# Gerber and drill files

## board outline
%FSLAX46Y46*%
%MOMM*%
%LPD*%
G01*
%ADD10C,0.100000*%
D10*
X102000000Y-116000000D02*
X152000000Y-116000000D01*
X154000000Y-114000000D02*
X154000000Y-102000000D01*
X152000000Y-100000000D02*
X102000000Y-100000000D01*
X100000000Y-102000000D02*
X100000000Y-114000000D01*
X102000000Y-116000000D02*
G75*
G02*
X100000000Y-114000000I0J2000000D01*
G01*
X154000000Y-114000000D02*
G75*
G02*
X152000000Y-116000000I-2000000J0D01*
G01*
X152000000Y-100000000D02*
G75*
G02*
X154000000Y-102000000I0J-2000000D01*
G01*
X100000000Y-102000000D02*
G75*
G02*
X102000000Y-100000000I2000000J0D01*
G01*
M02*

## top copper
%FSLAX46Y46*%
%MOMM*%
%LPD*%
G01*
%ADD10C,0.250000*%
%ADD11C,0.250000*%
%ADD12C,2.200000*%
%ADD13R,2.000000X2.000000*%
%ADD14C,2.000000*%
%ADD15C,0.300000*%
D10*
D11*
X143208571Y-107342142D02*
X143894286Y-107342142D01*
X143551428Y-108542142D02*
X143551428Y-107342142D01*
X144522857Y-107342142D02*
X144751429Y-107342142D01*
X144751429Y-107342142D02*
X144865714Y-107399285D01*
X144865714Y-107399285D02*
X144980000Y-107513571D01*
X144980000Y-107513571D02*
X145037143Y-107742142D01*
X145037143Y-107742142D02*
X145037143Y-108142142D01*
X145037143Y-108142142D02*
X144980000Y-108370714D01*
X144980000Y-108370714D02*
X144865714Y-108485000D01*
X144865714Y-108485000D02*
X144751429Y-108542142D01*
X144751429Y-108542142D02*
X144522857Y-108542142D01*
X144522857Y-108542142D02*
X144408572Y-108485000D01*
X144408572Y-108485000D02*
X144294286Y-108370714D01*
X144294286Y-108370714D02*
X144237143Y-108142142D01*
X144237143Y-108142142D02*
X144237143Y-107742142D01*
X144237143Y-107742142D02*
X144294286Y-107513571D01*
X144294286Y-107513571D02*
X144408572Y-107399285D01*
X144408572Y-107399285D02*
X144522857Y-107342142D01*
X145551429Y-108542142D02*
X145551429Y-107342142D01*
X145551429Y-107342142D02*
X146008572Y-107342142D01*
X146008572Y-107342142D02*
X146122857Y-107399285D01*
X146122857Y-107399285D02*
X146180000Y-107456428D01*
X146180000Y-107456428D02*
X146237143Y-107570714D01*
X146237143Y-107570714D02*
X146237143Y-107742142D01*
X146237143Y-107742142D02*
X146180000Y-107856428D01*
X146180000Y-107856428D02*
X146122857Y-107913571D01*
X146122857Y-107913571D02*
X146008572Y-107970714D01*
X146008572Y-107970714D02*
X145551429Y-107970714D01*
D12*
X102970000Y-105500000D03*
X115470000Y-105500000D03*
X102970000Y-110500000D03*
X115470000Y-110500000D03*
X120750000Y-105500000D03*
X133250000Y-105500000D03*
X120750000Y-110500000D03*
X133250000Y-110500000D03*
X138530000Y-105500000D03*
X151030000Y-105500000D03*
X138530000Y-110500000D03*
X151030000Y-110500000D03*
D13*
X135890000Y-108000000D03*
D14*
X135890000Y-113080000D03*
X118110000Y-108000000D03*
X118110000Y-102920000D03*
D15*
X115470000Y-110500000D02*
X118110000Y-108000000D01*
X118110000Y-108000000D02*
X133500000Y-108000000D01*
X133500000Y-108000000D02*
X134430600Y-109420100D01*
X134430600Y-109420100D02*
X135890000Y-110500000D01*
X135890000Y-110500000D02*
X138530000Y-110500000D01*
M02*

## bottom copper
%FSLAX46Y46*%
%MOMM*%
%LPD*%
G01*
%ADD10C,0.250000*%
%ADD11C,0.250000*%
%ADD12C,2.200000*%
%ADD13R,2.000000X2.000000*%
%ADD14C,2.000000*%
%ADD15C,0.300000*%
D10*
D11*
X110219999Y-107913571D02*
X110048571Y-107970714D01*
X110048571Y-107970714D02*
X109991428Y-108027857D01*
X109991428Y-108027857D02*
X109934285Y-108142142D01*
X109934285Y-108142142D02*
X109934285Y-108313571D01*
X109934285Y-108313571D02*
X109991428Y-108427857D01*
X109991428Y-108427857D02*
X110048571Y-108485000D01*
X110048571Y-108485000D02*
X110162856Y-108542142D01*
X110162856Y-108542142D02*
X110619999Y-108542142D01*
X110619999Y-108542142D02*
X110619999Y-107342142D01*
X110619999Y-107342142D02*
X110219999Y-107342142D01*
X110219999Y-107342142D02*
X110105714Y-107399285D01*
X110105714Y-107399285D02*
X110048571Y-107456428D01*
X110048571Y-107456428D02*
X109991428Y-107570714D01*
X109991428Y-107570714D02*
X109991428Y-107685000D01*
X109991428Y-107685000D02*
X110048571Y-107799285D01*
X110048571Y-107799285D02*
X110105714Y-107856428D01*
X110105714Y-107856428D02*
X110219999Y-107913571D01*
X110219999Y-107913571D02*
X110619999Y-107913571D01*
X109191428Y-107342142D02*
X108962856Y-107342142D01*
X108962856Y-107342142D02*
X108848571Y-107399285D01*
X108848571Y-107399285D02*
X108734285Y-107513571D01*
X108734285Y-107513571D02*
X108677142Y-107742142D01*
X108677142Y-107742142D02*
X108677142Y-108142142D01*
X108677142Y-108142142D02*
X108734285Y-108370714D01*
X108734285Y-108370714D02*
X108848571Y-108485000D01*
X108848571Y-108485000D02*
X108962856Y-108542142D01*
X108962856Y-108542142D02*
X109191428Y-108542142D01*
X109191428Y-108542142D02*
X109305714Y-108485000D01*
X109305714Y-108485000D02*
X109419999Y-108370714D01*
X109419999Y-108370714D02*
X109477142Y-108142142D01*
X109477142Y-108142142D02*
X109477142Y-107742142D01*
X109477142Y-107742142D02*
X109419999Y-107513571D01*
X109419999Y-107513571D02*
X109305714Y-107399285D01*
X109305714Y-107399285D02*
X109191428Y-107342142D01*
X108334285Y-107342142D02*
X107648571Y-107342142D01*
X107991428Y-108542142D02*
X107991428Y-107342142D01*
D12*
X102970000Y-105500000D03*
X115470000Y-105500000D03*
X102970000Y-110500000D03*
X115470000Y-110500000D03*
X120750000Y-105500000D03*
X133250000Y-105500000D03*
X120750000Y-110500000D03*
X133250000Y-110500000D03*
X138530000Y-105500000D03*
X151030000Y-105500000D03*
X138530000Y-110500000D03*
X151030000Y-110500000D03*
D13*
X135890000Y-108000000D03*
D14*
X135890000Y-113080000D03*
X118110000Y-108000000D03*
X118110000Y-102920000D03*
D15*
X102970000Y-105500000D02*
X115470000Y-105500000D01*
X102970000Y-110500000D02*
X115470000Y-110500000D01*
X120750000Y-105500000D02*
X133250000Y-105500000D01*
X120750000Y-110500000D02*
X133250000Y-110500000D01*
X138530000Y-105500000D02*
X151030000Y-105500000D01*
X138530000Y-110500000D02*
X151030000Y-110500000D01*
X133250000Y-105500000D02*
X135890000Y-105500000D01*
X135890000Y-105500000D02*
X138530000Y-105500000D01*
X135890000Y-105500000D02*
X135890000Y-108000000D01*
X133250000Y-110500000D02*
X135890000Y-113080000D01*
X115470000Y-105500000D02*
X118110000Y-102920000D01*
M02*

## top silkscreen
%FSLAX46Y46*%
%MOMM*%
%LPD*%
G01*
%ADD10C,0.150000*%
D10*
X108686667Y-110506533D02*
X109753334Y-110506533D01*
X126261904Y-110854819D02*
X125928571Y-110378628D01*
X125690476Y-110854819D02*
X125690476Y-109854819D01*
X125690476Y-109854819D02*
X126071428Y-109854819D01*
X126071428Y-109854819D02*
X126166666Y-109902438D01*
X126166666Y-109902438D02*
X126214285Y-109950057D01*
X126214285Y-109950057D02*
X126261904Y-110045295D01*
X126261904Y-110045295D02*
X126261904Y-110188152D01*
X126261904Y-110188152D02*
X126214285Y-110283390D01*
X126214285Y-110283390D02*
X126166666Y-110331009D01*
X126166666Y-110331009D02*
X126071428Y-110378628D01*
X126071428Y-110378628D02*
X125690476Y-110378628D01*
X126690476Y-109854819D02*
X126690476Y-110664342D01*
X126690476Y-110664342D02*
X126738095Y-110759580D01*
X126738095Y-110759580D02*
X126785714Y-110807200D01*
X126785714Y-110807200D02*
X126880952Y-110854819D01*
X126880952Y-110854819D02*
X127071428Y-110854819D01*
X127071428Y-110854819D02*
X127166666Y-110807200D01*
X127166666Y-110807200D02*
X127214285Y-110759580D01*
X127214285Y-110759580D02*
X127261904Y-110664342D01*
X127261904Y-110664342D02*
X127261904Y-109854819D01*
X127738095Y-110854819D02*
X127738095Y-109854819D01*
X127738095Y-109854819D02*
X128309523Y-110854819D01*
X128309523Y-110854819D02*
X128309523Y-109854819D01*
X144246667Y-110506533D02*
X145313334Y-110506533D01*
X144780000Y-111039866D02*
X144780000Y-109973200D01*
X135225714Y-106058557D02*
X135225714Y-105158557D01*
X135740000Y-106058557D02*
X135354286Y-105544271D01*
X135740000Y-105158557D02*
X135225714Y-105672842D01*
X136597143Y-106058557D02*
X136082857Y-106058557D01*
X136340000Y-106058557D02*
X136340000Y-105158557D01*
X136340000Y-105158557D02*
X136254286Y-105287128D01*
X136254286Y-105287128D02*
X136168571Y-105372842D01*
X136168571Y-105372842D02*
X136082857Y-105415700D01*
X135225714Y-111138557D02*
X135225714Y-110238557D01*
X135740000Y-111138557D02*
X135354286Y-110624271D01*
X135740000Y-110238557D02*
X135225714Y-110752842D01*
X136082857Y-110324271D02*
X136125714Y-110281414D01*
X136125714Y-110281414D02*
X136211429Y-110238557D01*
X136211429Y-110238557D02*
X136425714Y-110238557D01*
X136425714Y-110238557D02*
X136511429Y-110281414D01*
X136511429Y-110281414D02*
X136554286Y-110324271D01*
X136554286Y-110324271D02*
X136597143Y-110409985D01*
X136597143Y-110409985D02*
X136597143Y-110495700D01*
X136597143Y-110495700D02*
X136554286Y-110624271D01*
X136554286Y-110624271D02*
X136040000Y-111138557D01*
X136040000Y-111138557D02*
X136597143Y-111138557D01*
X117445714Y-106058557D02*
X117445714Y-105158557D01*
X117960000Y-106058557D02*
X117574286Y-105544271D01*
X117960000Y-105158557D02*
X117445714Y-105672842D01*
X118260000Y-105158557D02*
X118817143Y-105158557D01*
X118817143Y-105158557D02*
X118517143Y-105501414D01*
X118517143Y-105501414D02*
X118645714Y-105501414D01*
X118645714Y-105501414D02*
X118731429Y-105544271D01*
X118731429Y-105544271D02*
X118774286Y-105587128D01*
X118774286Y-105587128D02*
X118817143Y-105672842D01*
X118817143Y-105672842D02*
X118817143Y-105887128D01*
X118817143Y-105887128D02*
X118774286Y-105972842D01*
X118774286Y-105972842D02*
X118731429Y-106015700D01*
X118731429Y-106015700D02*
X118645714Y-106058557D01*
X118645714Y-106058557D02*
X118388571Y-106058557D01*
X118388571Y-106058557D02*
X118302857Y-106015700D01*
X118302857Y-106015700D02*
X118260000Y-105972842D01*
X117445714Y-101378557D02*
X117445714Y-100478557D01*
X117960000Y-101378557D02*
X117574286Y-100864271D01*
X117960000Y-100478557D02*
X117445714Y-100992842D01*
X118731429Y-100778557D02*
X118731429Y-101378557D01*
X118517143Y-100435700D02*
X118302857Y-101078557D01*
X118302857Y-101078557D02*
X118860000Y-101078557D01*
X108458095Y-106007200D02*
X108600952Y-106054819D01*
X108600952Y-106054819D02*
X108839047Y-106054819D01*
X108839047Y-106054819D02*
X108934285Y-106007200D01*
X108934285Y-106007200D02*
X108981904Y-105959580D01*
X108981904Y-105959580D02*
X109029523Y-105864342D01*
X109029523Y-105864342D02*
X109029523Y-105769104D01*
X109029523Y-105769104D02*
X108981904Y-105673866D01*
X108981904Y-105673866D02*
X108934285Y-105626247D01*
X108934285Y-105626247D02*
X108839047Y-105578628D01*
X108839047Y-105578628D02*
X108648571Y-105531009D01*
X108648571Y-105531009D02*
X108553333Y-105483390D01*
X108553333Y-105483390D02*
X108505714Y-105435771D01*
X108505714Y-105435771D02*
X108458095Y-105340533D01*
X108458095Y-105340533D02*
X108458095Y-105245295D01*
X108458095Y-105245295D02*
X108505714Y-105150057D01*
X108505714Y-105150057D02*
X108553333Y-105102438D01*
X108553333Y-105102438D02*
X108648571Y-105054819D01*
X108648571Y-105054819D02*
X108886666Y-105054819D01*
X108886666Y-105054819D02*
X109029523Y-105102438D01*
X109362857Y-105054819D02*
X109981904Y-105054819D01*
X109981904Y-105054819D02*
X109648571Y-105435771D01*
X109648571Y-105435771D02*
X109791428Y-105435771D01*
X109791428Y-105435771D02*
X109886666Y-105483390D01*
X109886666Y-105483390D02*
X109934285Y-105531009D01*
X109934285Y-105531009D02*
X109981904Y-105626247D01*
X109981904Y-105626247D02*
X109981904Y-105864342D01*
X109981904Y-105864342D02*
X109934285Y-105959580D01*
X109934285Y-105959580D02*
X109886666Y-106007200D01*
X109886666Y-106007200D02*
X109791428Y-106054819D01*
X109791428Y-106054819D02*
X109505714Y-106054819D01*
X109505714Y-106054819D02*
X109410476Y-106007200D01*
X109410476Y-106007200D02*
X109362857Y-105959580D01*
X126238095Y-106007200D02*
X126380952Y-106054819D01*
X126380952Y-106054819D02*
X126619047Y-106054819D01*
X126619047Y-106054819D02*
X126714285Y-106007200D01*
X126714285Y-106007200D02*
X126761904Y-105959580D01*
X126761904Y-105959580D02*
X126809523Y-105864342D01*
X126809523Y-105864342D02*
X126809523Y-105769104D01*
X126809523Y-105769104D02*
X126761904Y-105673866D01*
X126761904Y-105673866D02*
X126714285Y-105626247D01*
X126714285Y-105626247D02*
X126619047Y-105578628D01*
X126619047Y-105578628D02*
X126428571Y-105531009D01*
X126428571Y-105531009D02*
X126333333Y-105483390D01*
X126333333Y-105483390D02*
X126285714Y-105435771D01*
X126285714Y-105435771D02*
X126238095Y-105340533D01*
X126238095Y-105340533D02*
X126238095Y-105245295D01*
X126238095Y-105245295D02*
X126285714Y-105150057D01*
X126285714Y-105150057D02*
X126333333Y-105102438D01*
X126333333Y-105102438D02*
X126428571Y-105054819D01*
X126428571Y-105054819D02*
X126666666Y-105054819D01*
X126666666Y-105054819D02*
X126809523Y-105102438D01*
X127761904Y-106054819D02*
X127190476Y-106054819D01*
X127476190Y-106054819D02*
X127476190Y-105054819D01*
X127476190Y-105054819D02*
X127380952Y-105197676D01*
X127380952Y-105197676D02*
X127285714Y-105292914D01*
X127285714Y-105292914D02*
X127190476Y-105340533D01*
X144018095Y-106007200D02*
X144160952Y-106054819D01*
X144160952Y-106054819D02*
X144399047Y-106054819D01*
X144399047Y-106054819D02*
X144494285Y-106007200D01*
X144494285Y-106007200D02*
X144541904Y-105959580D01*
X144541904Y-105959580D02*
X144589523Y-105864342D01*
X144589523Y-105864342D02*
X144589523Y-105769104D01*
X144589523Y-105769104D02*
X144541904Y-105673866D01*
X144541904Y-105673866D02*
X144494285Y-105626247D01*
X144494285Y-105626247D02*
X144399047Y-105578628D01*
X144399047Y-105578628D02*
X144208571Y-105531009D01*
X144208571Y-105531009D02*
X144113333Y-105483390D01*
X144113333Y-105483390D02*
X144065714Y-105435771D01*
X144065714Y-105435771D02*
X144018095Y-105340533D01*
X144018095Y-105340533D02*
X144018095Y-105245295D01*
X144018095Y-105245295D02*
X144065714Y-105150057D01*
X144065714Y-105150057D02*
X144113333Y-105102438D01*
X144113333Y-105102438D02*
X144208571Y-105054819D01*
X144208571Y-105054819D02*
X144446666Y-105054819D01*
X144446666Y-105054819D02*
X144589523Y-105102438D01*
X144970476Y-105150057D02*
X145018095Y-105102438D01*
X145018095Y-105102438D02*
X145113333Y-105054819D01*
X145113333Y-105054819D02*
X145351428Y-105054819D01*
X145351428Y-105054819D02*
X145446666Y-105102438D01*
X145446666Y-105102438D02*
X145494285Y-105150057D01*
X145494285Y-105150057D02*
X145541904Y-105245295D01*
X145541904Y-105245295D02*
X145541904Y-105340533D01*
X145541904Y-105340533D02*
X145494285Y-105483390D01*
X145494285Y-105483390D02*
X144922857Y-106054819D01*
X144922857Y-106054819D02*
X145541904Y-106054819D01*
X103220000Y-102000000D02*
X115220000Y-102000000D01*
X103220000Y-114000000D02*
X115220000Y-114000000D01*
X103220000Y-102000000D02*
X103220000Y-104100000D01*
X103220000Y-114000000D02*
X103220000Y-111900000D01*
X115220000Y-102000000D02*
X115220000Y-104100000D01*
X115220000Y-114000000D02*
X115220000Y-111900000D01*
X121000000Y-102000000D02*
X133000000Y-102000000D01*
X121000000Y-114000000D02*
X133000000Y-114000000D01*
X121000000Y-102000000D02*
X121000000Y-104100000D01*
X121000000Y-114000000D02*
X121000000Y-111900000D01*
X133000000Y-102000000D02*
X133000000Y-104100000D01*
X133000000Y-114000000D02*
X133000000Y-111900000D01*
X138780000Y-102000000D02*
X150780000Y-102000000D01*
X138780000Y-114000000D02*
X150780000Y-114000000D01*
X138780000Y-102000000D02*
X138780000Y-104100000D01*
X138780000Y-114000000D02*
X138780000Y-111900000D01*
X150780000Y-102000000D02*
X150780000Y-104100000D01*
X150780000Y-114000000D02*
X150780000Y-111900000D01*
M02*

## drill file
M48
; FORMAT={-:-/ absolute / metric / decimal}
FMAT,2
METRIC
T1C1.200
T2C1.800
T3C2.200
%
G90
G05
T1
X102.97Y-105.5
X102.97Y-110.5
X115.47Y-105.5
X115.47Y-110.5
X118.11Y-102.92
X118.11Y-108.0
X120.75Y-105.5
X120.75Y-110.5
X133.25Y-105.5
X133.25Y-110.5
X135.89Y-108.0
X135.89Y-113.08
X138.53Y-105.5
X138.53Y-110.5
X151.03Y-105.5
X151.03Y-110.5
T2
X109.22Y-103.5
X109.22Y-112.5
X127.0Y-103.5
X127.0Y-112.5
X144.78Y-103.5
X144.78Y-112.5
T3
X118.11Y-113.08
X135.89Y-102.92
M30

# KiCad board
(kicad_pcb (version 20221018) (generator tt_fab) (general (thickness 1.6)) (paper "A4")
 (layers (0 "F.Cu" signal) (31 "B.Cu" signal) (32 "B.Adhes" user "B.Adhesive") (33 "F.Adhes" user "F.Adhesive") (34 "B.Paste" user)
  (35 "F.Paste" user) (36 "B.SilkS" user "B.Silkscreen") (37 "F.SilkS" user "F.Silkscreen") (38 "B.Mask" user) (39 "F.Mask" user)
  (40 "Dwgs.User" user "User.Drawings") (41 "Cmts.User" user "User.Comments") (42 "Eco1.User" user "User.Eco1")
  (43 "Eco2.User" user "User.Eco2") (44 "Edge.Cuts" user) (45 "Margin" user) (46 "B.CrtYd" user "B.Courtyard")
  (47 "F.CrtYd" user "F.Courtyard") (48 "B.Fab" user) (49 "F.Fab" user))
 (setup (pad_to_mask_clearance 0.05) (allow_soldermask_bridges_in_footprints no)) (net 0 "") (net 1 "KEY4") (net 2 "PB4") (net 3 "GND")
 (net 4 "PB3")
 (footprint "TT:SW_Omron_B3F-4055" (layer "F.Cu") (at 109.22 108)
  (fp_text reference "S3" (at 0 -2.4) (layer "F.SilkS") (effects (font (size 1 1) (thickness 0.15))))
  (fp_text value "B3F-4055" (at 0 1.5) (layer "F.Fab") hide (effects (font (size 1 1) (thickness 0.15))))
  (fp_line (start -6 -6) (end 6 -6) (stroke (width 0.15) (type solid)) (layer "F.SilkS"))
  (fp_line (start -6 6) (end 6 6) (stroke (width 0.15) (type solid)) (layer "F.SilkS"))
  (fp_line (start -6 -6) (end -6 -3.9) (stroke (width 0.15) (type solid)) (layer "F.SilkS"))
  (fp_line (start -6 6) (end -6 3.9) (stroke (width 0.15) (type solid)) (layer "F.SilkS"))
  (fp_line (start 6 -6) (end 6 -3.9) (stroke (width 0.15) (type solid)) (layer "F.SilkS"))
  (fp_line (start 6 6) (end 6 3.9) (stroke (width 0.15) (type solid)) (layer "F.SilkS"))
  (pad "4" thru_hole circle (at -6.25 -2.5) (size 2.2 2.2) (drill 1.2) (layers "*.Cu" "*.Mask") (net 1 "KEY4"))
  (pad "3" thru_hole circle (at 6.25 -2.5) (size 2.2 2.2) (drill 1.2) (layers "*.Cu" "*.Mask") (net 1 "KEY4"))
  (pad "2" thru_hole circle (at -6.25 2.5) (size 2.2 2.2) (drill 1.2) (layers "*.Cu" "*.Mask") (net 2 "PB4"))
  (pad "1" thru_hole circle (at 6.25 2.5) (size 2.2 2.2) (drill 1.2) (layers "*.Cu" "*.Mask") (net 2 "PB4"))
  (pad "" np_thru_hole circle (at 0 4.5) (size 1.8 1.8) (drill 1.8) (layers "*.Cu" "*.Mask"))
  (pad "" np_thru_hole circle (at 0 -4.5) (size 1.8 1.8) (drill 1.8) (layers "*.Cu" "*.Mask")))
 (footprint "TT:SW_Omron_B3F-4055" (layer "F.Cu") (at 127 108)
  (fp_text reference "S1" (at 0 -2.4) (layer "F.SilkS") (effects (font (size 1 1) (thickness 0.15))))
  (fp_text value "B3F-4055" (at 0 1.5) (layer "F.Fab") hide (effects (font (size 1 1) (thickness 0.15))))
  (fp_line (start -6 -6) (end 6 -6) (stroke (width 0.15) (type solid)) (layer "F.SilkS"))
  (fp_line (start -6 6) (end 6 6) (stroke (width 0.15) (type solid)) (layer "F.SilkS"))
  (fp_line (start -6 -6) (end -6 -3.9) (stroke (width 0.15) (type solid)) (layer "F.SilkS"))
  (fp_line (start -6 6) (end -6 3.9) (stroke (width 0.15) (type solid)) (layer "F.SilkS"))
  (fp_line (start 6 -6) (end 6 -3.9) (stroke (width 0.15) (type solid)) (layer "F.SilkS"))
  (fp_line (start 6 6) (end 6 3.9) (stroke (width 0.15) (type solid)) (layer "F.SilkS"))
  (pad "4" thru_hole circle (at -6.25 -2.5) (size 2.2 2.2) (drill 1.2) (layers "*.Cu" "*.Mask") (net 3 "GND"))
  (pad "3" thru_hole circle (at 6.25 -2.5) (size 2.2 2.2) (drill 1.2) (layers "*.Cu" "*.Mask") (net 3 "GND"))
  (pad "2" thru_hole circle (at -6.25 2.5) (size 2.2 2.2) (drill 1.2) (layers "*.Cu" "*.Mask") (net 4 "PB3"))
  (pad "1" thru_hole circle (at 6.25 2.5) (size 2.2 2.2) (drill 1.2) (layers "*.Cu" "*.Mask") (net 4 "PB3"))
  (pad "" np_thru_hole circle (at 0 4.5) (size 1.8 1.8) (drill 1.8) (layers "*.Cu" "*.Mask"))
  (pad "" np_thru_hole circle (at 0 -4.5) (size 1.8 1.8) (drill 1.8) (layers "*.Cu" "*.Mask")))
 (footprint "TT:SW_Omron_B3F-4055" (layer "F.Cu") (at 144.78 108)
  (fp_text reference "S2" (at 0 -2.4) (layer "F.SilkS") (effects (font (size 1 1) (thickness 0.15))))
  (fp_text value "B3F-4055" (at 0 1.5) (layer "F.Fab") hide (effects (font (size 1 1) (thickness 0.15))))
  (fp_line (start -6 -6) (end 6 -6) (stroke (width 0.15) (type solid)) (layer "F.SilkS"))
  (fp_line (start -6 6) (end 6 6) (stroke (width 0.15) (type solid)) (layer "F.SilkS"))
  (fp_line (start -6 -6) (end -6 -3.9) (stroke (width 0.15) (type solid)) (layer "F.SilkS"))
  (fp_line (start -6 6) (end -6 3.9) (stroke (width 0.15) (type solid)) (layer "F.SilkS"))
  (fp_line (start 6 -6) (end 6 -3.9) (stroke (width 0.15) (type solid)) (layer "F.SilkS"))
  (fp_line (start 6 6) (end 6 3.9) (stroke (width 0.15) (type solid)) (layer "F.SilkS"))
  (pad "4" thru_hole circle (at -6.25 -2.5) (size 2.2 2.2) (drill 1.2) (layers "*.Cu" "*.Mask") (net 3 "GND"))
  (pad "3" thru_hole circle (at 6.25 -2.5) (size 2.2 2.2) (drill 1.2) (layers "*.Cu" "*.Mask") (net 3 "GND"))
  (pad "2" thru_hole circle (at -6.25 2.5) (size 2.2 2.2) (drill 1.2) (layers "*.Cu" "*.Mask") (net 2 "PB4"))
  (pad "1" thru_hole circle (at 6.25 2.5) (size 2.2 2.2) (drill 1.2) (layers "*.Cu" "*.Mask") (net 2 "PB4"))
  (pad "" np_thru_hole circle (at 0 4.5) (size 1.8 1.8) (drill 1.8) (layers "*.Cu" "*.Mask"))
  (pad "" np_thru_hole circle (at 0 -4.5) (size 1.8 1.8) (drill 1.8) (layers "*.Cu" "*.Mask")))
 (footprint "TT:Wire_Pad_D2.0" (layer "F.Cu") (at 135.89 108)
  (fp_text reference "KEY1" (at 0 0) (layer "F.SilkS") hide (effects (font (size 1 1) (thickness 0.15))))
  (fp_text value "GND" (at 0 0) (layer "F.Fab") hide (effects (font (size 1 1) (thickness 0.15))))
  (pad "1" thru_hole rect (at 0 0) (size 2 2) (drill 1.2) (layers "*.Cu" "*.Mask") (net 3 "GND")))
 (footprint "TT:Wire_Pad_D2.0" (layer "F.Cu") (at 135.89 113.08)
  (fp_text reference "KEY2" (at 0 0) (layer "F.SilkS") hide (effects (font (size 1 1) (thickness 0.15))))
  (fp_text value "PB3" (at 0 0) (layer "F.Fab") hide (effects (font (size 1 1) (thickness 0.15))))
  (pad "1" thru_hole circle (at 0 0) (size 2 2) (drill 1.2) (layers "*.Cu" "*.Mask") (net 4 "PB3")))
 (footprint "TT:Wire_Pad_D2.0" (layer "F.Cu") (at 118.11 108)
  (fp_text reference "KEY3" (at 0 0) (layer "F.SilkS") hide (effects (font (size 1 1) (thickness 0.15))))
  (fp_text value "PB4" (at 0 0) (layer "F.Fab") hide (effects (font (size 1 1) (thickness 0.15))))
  (pad "1" thru_hole circle (at 0 0) (size 2 2) (drill 1.2) (layers "*.Cu" "*.Mask") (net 2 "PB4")))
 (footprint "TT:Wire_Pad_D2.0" (layer "F.Cu") (at 118.11 102.92)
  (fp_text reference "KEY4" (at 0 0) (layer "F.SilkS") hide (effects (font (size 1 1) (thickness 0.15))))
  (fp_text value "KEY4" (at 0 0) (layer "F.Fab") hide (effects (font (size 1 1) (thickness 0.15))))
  (pad "1" thru_hole circle (at 0 0) (size 2 2) (drill 1.2) (layers "*.Cu" "*.Mask") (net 1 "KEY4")))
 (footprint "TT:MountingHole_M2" (layer "F.Cu") (at 118.11 113.08)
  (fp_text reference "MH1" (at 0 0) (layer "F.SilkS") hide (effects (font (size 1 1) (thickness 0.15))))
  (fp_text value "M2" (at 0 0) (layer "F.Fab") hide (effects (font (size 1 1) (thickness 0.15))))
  (pad "" np_thru_hole circle (at 0 0) (size 2.2 2.2) (drill 2.2) (layers "*.Cu" "*.Mask")))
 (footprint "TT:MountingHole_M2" (layer "F.Cu") (at 135.89 102.92)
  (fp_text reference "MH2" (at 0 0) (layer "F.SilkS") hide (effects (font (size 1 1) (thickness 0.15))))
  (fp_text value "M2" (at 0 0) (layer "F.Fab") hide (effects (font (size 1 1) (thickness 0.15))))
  (pad "" np_thru_hole circle (at 0 0) (size 2.2 2.2) (drill 2.2) (layers "*.Cu" "*.Mask")))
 (gr_line (start 102 116) (end 152 116) (stroke (width 0.1) (type solid)) (layer "Edge.Cuts"))
 (gr_line (start 154 114) (end 154 102) (stroke (width 0.1) (type solid)) (layer "Edge.Cuts"))
 (gr_line (start 152 100) (end 102 100) (stroke (width 0.1) (type solid)) (layer "Edge.Cuts"))
 (gr_line (start 100 102) (end 100 114) (stroke (width 0.1) (type solid)) (layer "Edge.Cuts"))
 (gr_arc (start 100 114) (mid 100.5858 115.4142) (end 102 116) (stroke (width 0.1) (type solid)) (layer "Edge.Cuts"))
 (gr_arc (start 152 116) (mid 153.4142 115.4142) (end 154 114) (stroke (width 0.1) (type solid)) (layer "Edge.Cuts"))
 (gr_arc (start 154 102) (mid 153.4142 100.5858) (end 152 100) (stroke (width 0.1) (type solid)) (layer "Edge.Cuts"))
 (gr_arc (start 102 100) (mid 100.5858 100.5858) (end 100 102) (stroke (width 0.1) (type solid)) (layer "Edge.Cuts"))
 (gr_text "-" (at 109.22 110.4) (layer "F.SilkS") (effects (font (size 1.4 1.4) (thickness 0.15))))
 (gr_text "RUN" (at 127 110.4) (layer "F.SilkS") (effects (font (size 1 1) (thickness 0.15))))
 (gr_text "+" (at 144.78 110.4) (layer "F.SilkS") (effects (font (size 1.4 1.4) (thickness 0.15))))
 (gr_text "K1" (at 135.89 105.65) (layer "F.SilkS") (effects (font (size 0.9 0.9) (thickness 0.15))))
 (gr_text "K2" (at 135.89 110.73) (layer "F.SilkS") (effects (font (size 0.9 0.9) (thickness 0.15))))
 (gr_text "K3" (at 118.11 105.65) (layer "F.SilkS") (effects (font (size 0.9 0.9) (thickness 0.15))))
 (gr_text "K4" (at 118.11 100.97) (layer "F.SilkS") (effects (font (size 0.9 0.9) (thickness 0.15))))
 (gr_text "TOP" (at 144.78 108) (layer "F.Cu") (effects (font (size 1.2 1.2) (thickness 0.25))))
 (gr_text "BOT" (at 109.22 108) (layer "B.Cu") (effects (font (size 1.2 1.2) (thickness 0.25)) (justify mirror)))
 (segment (start 102.97 105.5) (end 115.47 105.5) (width 0.3) (layer "B.Cu") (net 1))
 (segment (start 102.97 110.5) (end 115.47 110.5) (width 0.3) (layer "B.Cu") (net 2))
 (segment (start 120.75 105.5) (end 133.25 105.5) (width 0.3) (layer "B.Cu") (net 3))
 (segment (start 120.75 110.5) (end 133.25 110.5) (width 0.3) (layer "B.Cu") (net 4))
 (segment (start 138.53 105.5) (end 151.03 105.5) (width 0.3) (layer "B.Cu") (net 3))
 (segment (start 138.53 110.5) (end 151.03 110.5) (width 0.3) (layer "B.Cu") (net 2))
 (segment (start 133.25 105.5) (end 135.89 105.5) (width 0.3) (layer "B.Cu") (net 3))
 (segment (start 135.89 105.5) (end 138.53 105.5) (width 0.3) (layer "B.Cu") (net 3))
 (segment (start 135.89 105.5) (end 135.89 108) (width 0.3) (layer "B.Cu") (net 3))
 (segment (start 133.25 110.5) (end 135.89 113.08) (width 0.3) (layer "B.Cu") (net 4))
 (segment (start 115.47 105.5) (end 118.11 102.92) (width 0.3) (layer "B.Cu") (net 1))
 (segment (start 115.47 110.5) (end 118.11 108) (width 0.3) (layer "F.Cu") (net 2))
 (segment (start 118.11 108) (end 133.5 108) (width 0.3) (layer "F.Cu") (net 2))
 (segment (start 133.5 108) (end 134.4306 109.4201) (width 0.3) (layer "F.Cu") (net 2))
 (segment (start 134.4306 109.4201) (end 135.89 110.5) (width 0.3) (layer "F.Cu") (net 2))
 (segment (start 135.89 110.5) (end 138.53 110.5) (width 0.3) (layer "F.Cu") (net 2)))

